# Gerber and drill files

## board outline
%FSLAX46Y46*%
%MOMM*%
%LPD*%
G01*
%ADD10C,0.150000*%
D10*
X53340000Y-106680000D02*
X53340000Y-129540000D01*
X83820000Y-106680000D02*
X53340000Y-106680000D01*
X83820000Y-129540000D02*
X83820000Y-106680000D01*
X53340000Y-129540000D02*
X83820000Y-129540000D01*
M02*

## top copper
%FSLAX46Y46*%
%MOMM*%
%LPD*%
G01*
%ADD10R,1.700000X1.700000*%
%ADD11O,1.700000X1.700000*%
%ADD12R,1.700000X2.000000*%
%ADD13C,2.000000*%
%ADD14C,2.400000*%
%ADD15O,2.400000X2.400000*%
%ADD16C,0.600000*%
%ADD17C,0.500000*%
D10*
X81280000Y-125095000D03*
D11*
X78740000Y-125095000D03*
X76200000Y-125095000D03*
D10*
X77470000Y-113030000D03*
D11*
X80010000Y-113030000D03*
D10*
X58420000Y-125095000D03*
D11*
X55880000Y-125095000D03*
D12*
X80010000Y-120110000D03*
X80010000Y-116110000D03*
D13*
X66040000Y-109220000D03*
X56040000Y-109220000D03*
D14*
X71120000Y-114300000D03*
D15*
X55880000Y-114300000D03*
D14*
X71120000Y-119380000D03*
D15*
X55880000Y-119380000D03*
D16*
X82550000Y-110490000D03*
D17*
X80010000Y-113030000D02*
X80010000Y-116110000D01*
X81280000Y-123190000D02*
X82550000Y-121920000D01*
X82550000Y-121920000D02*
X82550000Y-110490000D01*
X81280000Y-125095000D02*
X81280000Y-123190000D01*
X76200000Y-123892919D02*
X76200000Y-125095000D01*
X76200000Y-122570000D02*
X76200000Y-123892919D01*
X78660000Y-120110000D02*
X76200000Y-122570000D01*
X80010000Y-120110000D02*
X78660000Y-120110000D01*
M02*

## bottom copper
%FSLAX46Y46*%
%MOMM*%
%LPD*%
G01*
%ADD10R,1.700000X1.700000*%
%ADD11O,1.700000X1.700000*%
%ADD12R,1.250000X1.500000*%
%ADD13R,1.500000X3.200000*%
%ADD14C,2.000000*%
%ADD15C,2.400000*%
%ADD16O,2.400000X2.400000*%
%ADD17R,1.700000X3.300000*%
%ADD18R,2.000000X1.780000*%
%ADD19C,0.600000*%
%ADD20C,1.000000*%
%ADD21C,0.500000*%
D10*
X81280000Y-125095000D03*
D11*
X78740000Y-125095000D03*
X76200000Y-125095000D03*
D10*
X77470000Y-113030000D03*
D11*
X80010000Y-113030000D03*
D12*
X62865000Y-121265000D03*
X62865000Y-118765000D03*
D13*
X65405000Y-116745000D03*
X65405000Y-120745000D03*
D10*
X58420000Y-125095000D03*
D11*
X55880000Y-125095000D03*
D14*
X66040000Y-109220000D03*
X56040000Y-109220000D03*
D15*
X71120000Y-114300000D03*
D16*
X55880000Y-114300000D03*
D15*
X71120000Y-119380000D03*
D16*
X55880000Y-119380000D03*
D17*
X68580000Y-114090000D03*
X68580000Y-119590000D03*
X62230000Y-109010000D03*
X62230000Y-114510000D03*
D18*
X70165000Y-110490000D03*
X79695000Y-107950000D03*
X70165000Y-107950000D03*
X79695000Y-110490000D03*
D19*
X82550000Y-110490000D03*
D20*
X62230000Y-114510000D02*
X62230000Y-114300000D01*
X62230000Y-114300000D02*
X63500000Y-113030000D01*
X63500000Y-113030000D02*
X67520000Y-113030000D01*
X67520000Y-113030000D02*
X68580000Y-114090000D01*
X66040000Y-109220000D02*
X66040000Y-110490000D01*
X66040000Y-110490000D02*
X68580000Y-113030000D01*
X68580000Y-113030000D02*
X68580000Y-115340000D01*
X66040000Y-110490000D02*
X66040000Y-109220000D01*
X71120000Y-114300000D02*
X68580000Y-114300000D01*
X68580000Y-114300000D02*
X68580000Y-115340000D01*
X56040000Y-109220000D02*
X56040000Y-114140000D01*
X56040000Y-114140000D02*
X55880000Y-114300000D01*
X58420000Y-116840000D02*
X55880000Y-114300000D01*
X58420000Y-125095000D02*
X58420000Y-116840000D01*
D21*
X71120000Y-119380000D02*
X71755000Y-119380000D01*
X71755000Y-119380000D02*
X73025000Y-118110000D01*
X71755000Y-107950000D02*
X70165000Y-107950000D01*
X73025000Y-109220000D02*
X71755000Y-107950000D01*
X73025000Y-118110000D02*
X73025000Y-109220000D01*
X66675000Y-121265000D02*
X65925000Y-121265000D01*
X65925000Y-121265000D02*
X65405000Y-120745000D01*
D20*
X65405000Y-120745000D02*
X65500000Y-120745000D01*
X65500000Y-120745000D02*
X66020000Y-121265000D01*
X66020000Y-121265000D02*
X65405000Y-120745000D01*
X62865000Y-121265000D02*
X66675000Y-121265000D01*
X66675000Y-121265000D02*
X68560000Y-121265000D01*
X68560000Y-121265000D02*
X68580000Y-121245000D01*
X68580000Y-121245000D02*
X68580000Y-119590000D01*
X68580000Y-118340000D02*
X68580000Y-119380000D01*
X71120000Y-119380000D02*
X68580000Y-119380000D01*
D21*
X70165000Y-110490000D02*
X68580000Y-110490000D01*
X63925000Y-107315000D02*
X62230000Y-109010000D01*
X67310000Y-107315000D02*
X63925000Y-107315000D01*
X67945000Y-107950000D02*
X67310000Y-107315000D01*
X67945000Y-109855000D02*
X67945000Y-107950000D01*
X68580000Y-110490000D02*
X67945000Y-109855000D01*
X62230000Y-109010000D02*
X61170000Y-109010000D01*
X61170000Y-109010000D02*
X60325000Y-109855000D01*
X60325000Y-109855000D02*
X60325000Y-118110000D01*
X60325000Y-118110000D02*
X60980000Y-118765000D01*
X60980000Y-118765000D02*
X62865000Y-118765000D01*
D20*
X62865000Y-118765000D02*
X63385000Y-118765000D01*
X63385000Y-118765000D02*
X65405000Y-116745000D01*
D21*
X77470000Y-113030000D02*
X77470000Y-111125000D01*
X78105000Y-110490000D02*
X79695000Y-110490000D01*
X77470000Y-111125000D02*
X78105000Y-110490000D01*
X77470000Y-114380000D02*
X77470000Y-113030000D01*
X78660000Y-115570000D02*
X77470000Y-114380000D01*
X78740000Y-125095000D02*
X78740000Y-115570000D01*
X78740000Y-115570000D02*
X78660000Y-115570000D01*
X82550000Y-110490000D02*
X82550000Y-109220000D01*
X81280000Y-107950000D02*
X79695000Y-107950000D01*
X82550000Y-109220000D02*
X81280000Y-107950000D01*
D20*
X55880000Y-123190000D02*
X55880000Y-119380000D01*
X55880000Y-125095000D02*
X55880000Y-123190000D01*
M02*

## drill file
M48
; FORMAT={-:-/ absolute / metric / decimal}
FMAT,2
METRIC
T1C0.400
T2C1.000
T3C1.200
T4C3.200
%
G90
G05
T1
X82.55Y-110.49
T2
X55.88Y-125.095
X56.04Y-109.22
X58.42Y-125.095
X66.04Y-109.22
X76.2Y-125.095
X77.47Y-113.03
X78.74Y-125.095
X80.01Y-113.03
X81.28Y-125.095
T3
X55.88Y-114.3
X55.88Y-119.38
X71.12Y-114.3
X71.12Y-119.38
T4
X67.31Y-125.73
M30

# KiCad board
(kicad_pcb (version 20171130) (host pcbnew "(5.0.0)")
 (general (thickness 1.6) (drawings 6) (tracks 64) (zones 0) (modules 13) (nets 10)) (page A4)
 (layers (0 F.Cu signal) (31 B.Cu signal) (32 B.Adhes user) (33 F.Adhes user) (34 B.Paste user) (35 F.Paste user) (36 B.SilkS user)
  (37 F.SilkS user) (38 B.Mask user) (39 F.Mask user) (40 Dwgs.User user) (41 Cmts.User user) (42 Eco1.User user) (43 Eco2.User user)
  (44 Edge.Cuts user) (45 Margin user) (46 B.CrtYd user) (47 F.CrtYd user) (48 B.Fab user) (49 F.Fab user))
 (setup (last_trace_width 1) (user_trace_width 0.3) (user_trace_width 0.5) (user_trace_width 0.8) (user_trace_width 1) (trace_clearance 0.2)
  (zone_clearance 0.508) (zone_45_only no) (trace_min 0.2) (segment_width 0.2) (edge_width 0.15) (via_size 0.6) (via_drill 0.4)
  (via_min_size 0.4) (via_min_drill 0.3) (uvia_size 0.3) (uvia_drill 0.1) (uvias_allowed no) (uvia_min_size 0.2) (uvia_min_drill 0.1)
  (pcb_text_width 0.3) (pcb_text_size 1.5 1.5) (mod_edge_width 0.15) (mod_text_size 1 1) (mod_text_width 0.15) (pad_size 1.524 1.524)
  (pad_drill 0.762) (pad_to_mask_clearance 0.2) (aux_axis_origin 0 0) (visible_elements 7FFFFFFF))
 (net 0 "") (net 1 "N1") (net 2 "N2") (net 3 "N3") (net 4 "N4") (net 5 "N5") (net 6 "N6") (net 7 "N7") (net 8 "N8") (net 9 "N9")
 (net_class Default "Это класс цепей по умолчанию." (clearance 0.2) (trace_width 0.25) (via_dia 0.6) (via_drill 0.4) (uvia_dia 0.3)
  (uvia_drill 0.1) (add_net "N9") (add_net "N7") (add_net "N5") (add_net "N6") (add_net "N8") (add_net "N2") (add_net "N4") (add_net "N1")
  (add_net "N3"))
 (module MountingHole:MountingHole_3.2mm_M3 (layer F.Cu) (at 67.31 125.73)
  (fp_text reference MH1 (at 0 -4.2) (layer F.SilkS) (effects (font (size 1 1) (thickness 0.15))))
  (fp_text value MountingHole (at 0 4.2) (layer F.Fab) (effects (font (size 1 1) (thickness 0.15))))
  (pad 1 np_thru_hole circle (at 0 0) (size 3.2 3.2) (drill 3.2) (layers *.Cu *.Mask)))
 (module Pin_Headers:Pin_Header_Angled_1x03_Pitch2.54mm (layer F.Cu) (at 81.28 125.095 270)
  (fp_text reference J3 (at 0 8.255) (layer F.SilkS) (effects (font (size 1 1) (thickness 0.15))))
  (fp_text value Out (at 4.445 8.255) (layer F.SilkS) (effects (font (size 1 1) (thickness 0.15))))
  (pad 1 thru_hole rect (at 0 0 270) (size 1.7 1.7) (drill 1) (layers *.Cu *.Mask) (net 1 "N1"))
  (pad 2 thru_hole oval (at 0 2.54 270) (size 1.7 1.7) (drill 1) (layers *.Cu *.Mask) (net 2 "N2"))
  (pad 3 thru_hole oval (at 0 5.08 270) (size 1.7 1.7) (drill 1) (layers *.Cu *.Mask) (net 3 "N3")))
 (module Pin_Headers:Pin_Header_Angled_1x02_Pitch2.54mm (layer F.Cu) (at 77.47 113.03 90)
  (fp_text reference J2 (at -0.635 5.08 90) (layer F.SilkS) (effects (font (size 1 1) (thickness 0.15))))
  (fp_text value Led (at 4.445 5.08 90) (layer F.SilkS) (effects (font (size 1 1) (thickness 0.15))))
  (pad 1 thru_hole rect (at 0 0 90) (size 1.7 1.7) (drill 1) (layers *.Cu *.Mask) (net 2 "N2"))
  (pad 2 thru_hole oval (at 0 2.54 90) (size 1.7 1.7) (drill 1) (layers *.Cu *.Mask) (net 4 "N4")))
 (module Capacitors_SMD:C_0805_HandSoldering (layer B.Cu) (at 62.865 120.015 90)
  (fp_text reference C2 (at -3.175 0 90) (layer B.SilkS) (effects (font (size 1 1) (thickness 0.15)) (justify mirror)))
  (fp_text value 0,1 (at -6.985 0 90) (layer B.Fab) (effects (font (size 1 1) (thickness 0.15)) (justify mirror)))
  (pad 1 smd rect (at -1.25 0 90) (size 1.5 1.25) (layers B.Cu B.Paste B.Mask) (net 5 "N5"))
  (pad 2 smd rect (at 1.25 0 90) (size 1.5 1.25) (layers B.Cu B.Paste B.Mask) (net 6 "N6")))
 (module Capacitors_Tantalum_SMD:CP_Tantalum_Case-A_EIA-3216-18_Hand (layer B.Cu) (at 65.405 118.745 270)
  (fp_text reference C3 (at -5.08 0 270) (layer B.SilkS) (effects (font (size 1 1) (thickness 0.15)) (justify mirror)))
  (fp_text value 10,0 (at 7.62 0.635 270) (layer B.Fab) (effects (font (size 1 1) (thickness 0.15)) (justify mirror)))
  (pad 1 smd rect (at -2 0 270) (size 3.2 1.5) (layers B.Cu B.Paste B.Mask) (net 6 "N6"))
  (pad 2 smd rect (at 2 0 270) (size 3.2 1.5) (layers B.Cu B.Paste B.Mask) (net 5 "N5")))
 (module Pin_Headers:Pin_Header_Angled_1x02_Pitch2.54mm (layer F.Cu) (at 58.42 125.095 270)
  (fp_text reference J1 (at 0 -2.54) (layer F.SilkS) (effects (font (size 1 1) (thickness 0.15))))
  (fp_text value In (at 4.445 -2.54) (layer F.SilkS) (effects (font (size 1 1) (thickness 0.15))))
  (pad 1 thru_hole rect (at 0 0 270) (size 1.7 1.7) (drill 1) (layers *.Cu *.Mask) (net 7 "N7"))
  (pad 2 thru_hole oval (at 0 2.54 270) (size 1.7 1.7) (drill 1) (layers *.Cu *.Mask) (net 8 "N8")))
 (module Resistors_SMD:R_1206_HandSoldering (layer F.Cu) (at 80.01 118.11 90)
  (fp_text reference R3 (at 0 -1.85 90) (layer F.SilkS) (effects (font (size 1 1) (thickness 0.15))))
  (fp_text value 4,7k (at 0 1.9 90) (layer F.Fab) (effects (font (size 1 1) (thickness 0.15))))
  (pad 1 smd rect (at -2 0 90) (size 2 1.7) (layers F.Cu F.Paste F.Mask) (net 3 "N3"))
  (pad 2 smd rect (at 2 0 90) (size 2 1.7) (layers F.Cu F.Paste F.Mask) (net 4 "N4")))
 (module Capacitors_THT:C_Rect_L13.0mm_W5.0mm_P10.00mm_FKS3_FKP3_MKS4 (layer F.Cu) (at 66.04 109.22 180)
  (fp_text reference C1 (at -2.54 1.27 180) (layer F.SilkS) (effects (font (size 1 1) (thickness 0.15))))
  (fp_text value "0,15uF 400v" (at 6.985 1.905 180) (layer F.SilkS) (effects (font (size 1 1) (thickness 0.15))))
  (pad 1 thru_hole circle (at 0 0 180) (size 2 2) (drill 1) (layers *.Cu *.Mask) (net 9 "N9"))
  (pad 2 thru_hole circle (at 10 0 180) (size 2 2) (drill 1) (layers *.Cu *.Mask) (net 7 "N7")))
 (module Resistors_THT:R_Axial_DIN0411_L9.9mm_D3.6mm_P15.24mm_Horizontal (layer F.Cu) (at 71.12 114.3 180)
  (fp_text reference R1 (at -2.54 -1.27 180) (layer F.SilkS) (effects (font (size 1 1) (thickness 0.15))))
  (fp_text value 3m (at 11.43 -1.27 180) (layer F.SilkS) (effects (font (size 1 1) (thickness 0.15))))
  (pad 1 thru_hole circle (at 0 0 180) (size 2.4 2.4) (drill 1.2) (layers *.Cu *.Mask) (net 9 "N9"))
  (pad 2 thru_hole oval (at 15.24 0 180) (size 2.4 2.4) (drill 1.2) (layers *.Cu *.Mask) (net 7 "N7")))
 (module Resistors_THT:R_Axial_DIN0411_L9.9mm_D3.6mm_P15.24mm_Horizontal (layer F.Cu) (at 71.12 119.38 180)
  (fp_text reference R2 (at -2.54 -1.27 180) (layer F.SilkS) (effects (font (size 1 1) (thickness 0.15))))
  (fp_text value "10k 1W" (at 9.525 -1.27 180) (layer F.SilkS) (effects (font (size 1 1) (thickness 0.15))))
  (pad 1 thru_hole circle (at 0 0 180) (size 2.4 2.4) (drill 1.2) (layers *.Cu *.Mask) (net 5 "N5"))
  (pad 2 thru_hole oval (at 15.24 0 180) (size 2.4 2.4) (drill 1.2) (layers *.Cu *.Mask) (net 8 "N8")))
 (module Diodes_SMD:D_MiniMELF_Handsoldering (layer B.Cu) (at 68.58 116.84 270)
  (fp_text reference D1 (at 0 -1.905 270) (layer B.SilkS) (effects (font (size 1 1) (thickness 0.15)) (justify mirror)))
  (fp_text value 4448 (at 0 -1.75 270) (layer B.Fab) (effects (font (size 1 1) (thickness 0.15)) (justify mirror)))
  (pad 1 smd rect (at -2.75 0 270) (size 3.3 1.7) (layers B.Cu B.Paste B.Mask) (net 9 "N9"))
  (pad 2 smd rect (at 2.75 0 270) (size 3.3 1.7) (layers B.Cu B.Paste B.Mask) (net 5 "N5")))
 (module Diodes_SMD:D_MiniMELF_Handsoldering (layer B.Cu) (at 62.23 111.76 270)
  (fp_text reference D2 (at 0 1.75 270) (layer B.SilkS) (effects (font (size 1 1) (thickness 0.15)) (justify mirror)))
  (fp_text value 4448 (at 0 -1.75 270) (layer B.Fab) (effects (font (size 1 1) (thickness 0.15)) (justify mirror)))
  (pad 1 smd rect (at -2.75 0 270) (size 3.3 1.7) (layers B.Cu B.Paste B.Mask) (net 6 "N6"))
  (pad 2 smd rect (at 2.75 0 270) (size 3.3 1.7) (layers B.Cu B.Paste B.Mask) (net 9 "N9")))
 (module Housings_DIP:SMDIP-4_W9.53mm (layer B.Cu) (at 74.93 109.22)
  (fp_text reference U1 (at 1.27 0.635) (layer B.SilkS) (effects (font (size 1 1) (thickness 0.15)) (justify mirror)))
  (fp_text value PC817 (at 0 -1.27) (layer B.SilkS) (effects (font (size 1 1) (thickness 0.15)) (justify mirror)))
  (pad 1 smd rect (at -4.765 1.27) (size 2 1.78) (layers B.Cu B.Paste B.Mask) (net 6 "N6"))
  (pad 3 smd rect (at 4.765 -1.27) (size 2 1.78) (layers B.Cu B.Paste B.Mask) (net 1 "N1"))
  (pad 2 smd rect (at -4.765 -1.27) (size 2 1.78) (layers B.Cu B.Paste B.Mask) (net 5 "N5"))
  (pad 4 smd rect (at 4.765 1.27) (size 2 1.78) (layers B.Cu B.Paste B.Mask) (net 2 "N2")))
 (gr_line (start 53.34 106.68) (end 53.34 129.54) (angle 90) (layer Edge.Cuts) (width 0.15))
 (gr_line (start 83.82 106.68) (end 53.34 106.68) (angle 90) (layer Edge.Cuts) (width 0.15))
 (gr_line (start 83.82 129.54) (end 83.82 106.68) (angle 90) (layer Edge.Cuts) (width 0.15))
 (gr_line (start 53.34 129.54) (end 83.82 129.54) (angle 90) (layer Edge.Cuts) (width 0.15))
 (segment (start 62.23 114.51) (end 62.23 114.3) (width 1) (layer B.Cu) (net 9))
 (segment (start 62.23 114.3) (end 63.5 113.03) (width 1) (layer B.Cu) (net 9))
 (segment (start 63.5 113.03) (end 67.52 113.03) (width 1) (layer B.Cu) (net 9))
 (segment (start 67.52 113.03) (end 68.58 114.09) (width 1) (layer B.Cu) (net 9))
 (segment (start 66.04 109.22) (end 66.04 110.49) (width 1) (layer B.Cu) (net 9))
 (segment (start 66.04 110.49) (end 68.58 113.03) (width 1) (layer B.Cu) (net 9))
 (segment (start 68.58 113.03) (end 68.58 115.34) (width 1) (layer B.Cu) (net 9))
 (segment (start 66.04 110.49) (end 66.04 109.22) (width 1) (layer B.Cu) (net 9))
 (segment (start 71.12 114.3) (end 68.58 114.3) (width 1) (layer B.Cu) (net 9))
 (segment (start 68.58 114.3) (end 68.58 115.34) (width 1) (layer B.Cu) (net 9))
 (segment (start 56.04 109.22) (end 56.04 114.14) (width 1) (layer B.Cu) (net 7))
 (segment (start 56.04 114.14) (end 55.88 114.3) (width 1) (layer B.Cu) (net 7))
 (segment (start 58.42 116.84) (end 55.88 114.3) (width 1) (layer B.Cu) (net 7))
 (segment (start 58.42 125.095) (end 58.42 116.84) (width 1) (layer B.Cu) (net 7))
 (segment (start 71.12 119.38) (end 71.755 119.38) (width 0.5) (layer B.Cu) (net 5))
 (segment (start 71.755 119.38) (end 73.025 118.11) (width 0.5) (layer B.Cu) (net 5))
 (segment (start 71.755 107.95) (end 70.165 107.95) (width 0.5) (layer B.Cu) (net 5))
 (segment (start 73.025 109.22) (end 71.755 107.95) (width 0.5) (layer B.Cu) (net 5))
 (segment (start 73.025 118.11) (end 73.025 109.22) (width 0.5) (layer B.Cu) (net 5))
 (segment (start 66.675 121.265) (end 65.925 121.265) (width 0.5) (layer B.Cu) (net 5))
 (segment (start 65.925 121.265) (end 65.405 120.745) (width 0.5) (layer B.Cu) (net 5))
 (segment (start 65.405 120.745) (end 65.5 120.745) (width 1) (layer B.Cu) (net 5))
 (segment (start 65.5 120.745) (end 66.02 121.265) (width 1) (layer B.Cu) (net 5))
 (segment (start 66.02 121.265) (end 65.405 120.745) (width 1) (layer B.Cu) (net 5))
 (segment (start 62.865 121.265) (end 66.675 121.265) (width 1) (layer B.Cu) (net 5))
 (segment (start 66.675 121.265) (end 68.56 121.265) (width 1) (layer B.Cu) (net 5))
 (segment (start 68.56 121.265) (end 68.58 121.245) (width 1) (layer B.Cu) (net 5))
 (segment (start 68.58 121.245) (end 68.58 119.59) (width 1) (layer B.Cu) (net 5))
 (segment (start 68.58 118.34) (end 68.58 119.38) (width 1) (layer B.Cu) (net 5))
 (segment (start 71.12 119.38) (end 68.58 119.38) (width 1) (layer B.Cu) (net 5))
 (segment (start 70.165 110.49) (end 68.58 110.49) (width 0.5) (layer B.Cu) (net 6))
 (segment (start 63.925 107.315) (end 62.23 109.01) (width 0.5) (layer B.Cu) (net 6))
 (segment (start 67.31 107.315) (end 63.925 107.315) (width 0.5) (layer B.Cu) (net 6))
 (segment (start 67.945 107.95) (end 67.31 107.315) (width 0.5) (layer B.Cu) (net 6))
 (segment (start 67.945 109.855) (end 67.945 107.95) (width 0.5) (layer B.Cu) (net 6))
 (segment (start 68.58 110.49) (end 67.945 109.855) (width 0.5) (layer B.Cu) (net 6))
 (segment (start 62.23 109.01) (end 61.17 109.01) (width 0.5) (layer B.Cu) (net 6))
 (segment (start 61.17 109.01) (end 60.325 109.855) (width 0.5) (layer B.Cu) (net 6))
 (segment (start 60.325 109.855) (end 60.325 118.11) (width 0.5) (layer B.Cu) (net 6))
 (segment (start 60.325 118.11) (end 60.98 118.765) (width 0.5) (layer B.Cu) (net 6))
 (segment (start 60.98 118.765) (end 62.865 118.765) (width 0.5) (layer B.Cu) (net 6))
 (segment (start 62.865 118.765) (end 63.385 118.765) (width 1) (layer B.Cu) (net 6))
 (segment (start 63.385 118.765) (end 65.405 116.745) (width 1) (layer B.Cu) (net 6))
 (segment (start 77.47 113.03) (end 77.47 111.125) (width 0.5) (layer B.Cu) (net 2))
 (segment (start 78.105 110.49) (end 79.695 110.49) (width 0.5) (layer B.Cu) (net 2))
 (segment (start 77.47 111.125) (end 78.105 110.49) (width 0.5) (layer B.Cu) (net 2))
 (segment (start 77.47 114.38) (end 77.47 113.03) (width 0.5) (layer B.Cu) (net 2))
 (segment (start 78.66 115.57) (end 77.47 114.38) (width 0.5) (layer B.Cu) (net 2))
 (segment (start 78.74 125.095) (end 78.74 115.57) (width 0.5) (layer B.Cu) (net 2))
 (segment (start 78.74 115.57) (end 78.66 115.57) (width 0.5) (layer B.Cu) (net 2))
 (segment (start 80.01 113.03) (end 80.01 116.11) (width 0.5) (layer F.Cu) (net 4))
 (segment (start 81.28 123.19) (end 82.55 121.92) (width 0.5) (layer F.Cu) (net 1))
 (via (at 82.55 110.49) (size 0.6) (drill 0.4) (layers F.Cu B.Cu) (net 1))
 (segment (start 82.55 121.92) (end 82.55 110.49) (width 0.5) (layer F.Cu) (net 1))
 (segment (start 82.55 110.49) (end 82.55 109.22) (width 0.5) (layer B.Cu) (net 1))
 (segment (start 81.28 107.95) (end 79.695 107.95) (width 0.5) (layer B.Cu) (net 1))
 (segment (start 82.55 109.22) (end 81.28 107.95) (width 0.5) (layer B.Cu) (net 1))
 (segment (start 81.28 125.095) (end 81.28 123.19) (width 0.5) (layer F.Cu) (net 1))
 (segment (start 76.2 123.892919) (end 76.2 125.095) (width 0.5) (layer F.Cu) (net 3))
 (segment (start 76.2 122.57) (end 76.2 123.892919) (width 0.5) (layer F.Cu) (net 3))
 (segment (start 78.66 120.11) (end 76.2 122.57) (width 0.5) (layer F.Cu) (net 3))
 (segment (start 80.01 120.11) (end 78.66 120.11) (width 0.5) (layer F.Cu) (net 3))
 (segment (start 55.88 123.19) (end 55.88 119.38) (width 1) (layer B.Cu) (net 8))
 (segment (start 55.88 125.095) (end 55.88 123.19) (width 1) (layer B.Cu) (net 8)))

